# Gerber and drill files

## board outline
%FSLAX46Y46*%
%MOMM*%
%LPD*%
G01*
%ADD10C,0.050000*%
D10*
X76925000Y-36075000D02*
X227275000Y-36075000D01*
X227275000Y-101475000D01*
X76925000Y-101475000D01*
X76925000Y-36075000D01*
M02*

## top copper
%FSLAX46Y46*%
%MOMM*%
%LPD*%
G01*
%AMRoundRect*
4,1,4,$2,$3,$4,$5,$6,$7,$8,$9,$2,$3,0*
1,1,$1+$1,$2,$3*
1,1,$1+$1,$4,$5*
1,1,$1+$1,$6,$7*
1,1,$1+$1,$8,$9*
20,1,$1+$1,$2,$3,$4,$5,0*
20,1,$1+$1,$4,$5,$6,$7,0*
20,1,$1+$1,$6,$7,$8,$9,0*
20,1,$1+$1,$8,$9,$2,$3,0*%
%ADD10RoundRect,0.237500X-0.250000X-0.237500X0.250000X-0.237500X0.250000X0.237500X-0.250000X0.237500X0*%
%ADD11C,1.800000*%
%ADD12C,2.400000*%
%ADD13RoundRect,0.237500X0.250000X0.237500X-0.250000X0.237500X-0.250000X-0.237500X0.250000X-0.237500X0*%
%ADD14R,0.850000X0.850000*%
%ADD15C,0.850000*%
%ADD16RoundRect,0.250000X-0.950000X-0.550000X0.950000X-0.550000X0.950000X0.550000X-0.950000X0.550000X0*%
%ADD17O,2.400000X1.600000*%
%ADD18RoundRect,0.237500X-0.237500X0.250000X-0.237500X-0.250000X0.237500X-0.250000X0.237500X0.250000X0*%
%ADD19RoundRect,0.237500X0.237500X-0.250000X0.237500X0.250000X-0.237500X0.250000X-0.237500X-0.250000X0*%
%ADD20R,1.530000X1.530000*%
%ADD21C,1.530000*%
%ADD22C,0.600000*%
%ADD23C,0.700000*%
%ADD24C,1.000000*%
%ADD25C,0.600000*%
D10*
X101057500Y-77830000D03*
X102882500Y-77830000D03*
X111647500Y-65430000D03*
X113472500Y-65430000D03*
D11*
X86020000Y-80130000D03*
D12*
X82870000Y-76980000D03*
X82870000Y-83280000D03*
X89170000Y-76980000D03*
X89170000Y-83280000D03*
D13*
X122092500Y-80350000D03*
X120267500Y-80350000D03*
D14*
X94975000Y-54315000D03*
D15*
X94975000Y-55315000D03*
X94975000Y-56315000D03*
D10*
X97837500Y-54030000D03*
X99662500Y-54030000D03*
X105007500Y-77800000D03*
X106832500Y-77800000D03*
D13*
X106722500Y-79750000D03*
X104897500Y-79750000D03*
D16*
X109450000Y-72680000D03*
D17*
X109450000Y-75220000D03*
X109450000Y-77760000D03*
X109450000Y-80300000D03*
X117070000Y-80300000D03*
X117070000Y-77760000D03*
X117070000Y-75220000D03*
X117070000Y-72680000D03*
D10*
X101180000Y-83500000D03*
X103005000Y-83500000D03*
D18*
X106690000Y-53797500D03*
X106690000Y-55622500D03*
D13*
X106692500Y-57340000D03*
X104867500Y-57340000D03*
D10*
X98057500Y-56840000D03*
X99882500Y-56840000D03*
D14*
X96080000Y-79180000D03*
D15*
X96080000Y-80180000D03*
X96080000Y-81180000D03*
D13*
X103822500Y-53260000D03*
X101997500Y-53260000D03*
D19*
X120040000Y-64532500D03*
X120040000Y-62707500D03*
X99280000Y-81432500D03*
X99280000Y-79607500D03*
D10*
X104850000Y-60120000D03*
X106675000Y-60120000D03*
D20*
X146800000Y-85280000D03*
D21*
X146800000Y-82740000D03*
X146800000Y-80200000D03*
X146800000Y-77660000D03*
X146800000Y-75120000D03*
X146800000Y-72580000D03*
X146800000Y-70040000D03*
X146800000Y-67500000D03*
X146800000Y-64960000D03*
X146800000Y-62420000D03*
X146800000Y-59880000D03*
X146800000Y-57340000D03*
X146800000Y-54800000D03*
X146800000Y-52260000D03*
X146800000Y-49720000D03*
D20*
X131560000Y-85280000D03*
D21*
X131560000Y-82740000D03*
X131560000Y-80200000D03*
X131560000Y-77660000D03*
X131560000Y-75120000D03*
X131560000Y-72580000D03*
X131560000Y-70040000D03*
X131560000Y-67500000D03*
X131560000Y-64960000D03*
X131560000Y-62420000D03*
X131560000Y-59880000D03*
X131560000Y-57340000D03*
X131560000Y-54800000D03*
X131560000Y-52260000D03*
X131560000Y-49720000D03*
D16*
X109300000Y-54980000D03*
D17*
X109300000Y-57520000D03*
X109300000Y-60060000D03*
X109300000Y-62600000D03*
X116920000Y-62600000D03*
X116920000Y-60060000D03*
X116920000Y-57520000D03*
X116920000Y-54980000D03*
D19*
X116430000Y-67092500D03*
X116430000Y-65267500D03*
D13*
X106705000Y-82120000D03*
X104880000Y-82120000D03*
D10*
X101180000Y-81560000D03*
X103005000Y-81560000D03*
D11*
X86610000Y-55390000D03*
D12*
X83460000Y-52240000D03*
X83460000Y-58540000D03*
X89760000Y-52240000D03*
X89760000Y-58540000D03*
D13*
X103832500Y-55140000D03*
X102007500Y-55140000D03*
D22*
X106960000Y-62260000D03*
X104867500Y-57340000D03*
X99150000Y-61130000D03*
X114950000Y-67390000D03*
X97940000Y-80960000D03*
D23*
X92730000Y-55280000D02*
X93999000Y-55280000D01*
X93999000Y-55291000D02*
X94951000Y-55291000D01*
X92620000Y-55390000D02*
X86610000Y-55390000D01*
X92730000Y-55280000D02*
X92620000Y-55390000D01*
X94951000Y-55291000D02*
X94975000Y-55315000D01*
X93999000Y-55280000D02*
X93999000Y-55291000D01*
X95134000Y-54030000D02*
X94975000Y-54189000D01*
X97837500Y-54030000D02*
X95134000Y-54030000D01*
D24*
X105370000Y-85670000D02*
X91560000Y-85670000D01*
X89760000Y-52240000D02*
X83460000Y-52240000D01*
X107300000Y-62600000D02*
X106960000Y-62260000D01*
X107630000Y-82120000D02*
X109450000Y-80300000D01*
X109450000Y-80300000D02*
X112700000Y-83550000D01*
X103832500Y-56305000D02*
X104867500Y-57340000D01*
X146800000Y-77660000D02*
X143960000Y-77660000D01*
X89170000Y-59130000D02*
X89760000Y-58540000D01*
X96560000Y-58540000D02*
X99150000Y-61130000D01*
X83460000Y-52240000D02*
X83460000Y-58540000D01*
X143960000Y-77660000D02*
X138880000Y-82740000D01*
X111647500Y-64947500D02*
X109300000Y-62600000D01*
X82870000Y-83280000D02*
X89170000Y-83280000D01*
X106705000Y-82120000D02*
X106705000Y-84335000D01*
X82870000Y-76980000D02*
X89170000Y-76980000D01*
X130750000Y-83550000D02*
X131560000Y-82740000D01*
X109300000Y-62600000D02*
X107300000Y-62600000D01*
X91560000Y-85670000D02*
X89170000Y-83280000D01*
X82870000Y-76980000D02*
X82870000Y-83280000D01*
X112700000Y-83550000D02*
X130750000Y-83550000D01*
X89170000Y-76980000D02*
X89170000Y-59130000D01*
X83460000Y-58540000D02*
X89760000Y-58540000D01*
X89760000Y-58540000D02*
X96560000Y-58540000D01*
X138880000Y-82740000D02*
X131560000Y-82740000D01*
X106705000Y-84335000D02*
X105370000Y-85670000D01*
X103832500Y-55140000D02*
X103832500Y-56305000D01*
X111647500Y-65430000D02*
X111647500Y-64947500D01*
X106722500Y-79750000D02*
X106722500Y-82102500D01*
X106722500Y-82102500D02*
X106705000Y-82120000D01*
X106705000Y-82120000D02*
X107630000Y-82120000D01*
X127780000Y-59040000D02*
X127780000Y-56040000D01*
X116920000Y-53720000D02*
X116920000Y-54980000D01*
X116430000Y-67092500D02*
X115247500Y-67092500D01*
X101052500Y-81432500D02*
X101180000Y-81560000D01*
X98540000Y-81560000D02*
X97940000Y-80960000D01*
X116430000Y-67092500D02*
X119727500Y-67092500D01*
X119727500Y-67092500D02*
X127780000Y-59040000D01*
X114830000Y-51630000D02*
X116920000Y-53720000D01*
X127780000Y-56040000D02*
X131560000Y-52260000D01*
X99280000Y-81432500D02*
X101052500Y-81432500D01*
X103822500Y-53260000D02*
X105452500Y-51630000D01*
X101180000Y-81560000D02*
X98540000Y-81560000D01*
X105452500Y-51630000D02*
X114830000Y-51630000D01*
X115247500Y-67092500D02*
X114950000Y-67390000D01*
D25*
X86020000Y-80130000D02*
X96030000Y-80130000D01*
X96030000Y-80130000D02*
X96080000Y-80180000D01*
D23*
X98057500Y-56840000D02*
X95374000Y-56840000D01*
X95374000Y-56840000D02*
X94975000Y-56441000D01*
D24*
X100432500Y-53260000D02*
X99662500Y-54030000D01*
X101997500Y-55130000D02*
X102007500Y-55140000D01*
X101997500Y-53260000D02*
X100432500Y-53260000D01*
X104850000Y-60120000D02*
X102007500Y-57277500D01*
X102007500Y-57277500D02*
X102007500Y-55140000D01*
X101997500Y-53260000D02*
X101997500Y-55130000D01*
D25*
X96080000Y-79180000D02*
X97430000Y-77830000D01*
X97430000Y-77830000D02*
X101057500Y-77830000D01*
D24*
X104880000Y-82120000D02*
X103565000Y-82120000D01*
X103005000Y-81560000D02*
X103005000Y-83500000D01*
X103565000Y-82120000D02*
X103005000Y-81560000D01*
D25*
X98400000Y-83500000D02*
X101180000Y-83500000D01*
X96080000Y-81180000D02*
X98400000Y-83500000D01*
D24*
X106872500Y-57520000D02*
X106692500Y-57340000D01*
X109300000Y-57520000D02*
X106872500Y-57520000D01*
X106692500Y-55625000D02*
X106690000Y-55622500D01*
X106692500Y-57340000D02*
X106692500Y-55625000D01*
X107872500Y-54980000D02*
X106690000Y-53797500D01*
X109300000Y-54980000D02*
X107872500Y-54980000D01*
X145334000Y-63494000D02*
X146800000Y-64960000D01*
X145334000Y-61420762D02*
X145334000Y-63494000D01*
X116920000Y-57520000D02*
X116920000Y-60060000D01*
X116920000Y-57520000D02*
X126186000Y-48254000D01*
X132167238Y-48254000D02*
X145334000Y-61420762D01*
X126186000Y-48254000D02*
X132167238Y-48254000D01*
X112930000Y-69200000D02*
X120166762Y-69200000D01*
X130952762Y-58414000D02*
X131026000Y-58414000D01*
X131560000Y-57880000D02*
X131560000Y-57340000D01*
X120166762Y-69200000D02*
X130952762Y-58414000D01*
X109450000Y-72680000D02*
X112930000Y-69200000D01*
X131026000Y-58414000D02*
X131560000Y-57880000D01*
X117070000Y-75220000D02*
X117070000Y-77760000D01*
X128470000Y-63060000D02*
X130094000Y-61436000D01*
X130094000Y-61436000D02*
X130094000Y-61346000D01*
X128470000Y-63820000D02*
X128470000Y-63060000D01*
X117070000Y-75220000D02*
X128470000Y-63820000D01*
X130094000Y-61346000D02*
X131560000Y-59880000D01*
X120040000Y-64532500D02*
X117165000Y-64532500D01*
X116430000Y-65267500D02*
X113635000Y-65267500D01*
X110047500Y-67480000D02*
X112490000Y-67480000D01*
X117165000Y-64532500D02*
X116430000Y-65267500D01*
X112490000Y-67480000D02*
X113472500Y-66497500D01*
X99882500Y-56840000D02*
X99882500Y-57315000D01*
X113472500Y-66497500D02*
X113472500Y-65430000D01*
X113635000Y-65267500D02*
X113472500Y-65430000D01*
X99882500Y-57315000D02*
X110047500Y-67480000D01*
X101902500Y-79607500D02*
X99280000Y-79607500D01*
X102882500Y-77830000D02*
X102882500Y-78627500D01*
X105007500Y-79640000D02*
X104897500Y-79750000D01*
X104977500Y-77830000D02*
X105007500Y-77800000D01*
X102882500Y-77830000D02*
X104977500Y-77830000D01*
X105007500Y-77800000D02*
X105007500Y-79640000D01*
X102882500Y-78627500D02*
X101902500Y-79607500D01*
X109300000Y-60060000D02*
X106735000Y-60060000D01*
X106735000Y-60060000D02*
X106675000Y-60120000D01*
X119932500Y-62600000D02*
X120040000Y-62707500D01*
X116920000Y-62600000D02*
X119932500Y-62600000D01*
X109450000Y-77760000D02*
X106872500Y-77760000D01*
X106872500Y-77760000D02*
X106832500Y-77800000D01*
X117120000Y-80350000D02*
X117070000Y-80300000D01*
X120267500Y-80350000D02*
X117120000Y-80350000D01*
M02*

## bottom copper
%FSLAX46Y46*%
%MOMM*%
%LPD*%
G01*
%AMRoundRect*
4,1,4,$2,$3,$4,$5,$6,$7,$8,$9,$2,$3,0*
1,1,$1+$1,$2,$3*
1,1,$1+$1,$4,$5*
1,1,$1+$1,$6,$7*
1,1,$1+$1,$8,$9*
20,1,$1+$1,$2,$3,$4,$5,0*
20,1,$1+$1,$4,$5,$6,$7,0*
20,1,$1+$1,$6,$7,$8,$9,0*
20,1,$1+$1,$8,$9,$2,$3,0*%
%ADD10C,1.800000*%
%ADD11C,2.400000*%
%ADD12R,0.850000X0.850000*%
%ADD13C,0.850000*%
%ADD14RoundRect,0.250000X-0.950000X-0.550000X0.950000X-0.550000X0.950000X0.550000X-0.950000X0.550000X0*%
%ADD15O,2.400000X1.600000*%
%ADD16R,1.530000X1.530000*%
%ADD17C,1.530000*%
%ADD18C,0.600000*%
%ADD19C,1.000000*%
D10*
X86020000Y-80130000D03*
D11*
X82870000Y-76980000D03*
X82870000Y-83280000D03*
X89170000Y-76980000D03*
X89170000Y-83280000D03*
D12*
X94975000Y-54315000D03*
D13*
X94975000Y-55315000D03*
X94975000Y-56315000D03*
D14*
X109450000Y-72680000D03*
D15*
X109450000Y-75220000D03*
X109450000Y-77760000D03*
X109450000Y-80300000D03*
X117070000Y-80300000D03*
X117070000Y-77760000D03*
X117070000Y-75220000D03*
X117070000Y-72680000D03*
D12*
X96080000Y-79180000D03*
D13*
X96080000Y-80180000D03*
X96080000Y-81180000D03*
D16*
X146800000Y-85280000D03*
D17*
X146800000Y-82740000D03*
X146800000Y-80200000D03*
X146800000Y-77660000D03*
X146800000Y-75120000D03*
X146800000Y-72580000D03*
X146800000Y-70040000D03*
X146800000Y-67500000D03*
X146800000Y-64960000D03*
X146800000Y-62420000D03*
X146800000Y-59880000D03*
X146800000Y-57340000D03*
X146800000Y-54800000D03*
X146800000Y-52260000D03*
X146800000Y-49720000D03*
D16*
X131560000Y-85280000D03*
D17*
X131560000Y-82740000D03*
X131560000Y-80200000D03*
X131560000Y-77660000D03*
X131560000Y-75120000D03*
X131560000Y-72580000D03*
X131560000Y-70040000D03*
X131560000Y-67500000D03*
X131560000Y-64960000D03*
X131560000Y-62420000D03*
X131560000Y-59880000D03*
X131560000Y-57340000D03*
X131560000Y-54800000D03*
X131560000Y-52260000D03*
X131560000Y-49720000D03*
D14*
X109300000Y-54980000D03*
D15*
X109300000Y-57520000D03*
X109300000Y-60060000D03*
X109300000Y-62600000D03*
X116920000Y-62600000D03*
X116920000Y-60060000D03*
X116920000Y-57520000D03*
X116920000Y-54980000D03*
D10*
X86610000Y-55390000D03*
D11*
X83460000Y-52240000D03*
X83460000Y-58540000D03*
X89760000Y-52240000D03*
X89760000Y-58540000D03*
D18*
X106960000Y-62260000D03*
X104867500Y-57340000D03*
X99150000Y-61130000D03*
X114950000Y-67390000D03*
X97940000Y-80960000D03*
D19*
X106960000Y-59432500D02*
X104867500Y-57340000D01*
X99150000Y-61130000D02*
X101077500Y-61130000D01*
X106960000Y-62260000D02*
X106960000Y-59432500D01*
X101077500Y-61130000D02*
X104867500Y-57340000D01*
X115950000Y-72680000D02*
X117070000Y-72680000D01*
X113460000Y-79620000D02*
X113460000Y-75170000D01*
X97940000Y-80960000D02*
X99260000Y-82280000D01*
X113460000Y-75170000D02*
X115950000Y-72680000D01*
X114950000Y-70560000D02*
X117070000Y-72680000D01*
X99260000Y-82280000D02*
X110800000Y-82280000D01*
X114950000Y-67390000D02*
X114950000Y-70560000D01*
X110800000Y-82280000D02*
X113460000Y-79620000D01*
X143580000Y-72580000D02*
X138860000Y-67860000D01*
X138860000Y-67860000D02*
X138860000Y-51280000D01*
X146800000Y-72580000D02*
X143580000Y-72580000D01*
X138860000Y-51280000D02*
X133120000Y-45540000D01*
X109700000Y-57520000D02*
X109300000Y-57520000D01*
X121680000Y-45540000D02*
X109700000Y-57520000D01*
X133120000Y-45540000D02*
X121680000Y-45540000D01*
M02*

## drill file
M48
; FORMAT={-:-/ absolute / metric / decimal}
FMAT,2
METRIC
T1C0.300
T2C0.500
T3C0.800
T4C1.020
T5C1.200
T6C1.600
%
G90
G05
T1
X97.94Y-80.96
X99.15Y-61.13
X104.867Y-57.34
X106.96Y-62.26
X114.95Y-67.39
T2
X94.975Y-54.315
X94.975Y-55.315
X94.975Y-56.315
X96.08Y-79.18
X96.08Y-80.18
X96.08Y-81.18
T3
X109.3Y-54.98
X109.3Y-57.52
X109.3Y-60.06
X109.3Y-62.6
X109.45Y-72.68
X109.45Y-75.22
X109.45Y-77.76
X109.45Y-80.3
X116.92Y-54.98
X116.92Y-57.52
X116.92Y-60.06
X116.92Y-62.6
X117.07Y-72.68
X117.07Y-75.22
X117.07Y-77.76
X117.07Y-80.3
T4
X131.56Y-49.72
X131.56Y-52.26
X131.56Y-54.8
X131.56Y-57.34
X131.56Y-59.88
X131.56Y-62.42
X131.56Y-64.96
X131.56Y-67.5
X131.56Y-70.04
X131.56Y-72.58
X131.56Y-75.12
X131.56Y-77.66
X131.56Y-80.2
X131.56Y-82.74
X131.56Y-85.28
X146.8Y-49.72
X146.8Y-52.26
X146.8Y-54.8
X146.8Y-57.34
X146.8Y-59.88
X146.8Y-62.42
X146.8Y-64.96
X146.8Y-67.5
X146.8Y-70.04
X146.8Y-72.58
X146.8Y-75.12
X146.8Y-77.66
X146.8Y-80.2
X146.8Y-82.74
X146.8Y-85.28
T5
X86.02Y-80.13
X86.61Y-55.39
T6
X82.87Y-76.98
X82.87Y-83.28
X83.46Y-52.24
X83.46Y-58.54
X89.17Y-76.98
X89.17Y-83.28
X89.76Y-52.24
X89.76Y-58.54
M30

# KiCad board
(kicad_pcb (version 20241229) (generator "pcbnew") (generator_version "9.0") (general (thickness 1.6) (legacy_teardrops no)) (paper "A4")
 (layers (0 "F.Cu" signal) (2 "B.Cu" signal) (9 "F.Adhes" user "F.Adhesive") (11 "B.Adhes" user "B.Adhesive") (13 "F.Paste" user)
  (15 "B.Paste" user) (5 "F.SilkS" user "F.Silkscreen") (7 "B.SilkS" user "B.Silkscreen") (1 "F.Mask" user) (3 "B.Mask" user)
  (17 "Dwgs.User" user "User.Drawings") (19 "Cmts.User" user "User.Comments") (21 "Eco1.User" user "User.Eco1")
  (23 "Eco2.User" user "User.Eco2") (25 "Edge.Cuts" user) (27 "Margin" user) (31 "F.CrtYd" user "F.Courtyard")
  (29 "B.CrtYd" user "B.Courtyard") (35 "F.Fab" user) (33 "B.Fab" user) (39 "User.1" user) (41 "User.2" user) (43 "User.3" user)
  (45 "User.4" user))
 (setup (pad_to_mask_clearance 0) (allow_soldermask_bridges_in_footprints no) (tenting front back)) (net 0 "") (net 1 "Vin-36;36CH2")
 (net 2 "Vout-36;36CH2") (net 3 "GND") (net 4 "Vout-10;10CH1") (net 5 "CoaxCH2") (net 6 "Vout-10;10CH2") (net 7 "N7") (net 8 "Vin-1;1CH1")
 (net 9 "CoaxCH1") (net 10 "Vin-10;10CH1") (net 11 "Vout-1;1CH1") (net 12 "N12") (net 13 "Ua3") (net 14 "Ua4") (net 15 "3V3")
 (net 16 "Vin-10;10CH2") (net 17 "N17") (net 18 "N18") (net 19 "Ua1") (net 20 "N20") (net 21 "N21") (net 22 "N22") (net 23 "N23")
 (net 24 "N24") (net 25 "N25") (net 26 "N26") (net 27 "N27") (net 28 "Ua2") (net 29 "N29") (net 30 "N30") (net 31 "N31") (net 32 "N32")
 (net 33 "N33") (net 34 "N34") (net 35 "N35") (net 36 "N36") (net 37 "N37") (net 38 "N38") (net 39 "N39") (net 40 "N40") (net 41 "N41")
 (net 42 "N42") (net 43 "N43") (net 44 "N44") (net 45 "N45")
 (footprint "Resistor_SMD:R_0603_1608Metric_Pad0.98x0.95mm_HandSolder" (layer "F.Cu") (at 101.97 77.83)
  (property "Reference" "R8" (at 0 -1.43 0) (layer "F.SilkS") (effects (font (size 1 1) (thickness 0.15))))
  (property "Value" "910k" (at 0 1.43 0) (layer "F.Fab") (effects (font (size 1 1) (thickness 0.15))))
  (pad "1" smd roundrect (at -0.9125 0) (size 0.975 0.95) (layers "F.Cu" "F.Mask" "F.Paste") (roundrect_rratio 0.25) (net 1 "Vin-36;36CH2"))
  (pad "2" smd roundrect (at 0.9125 0) (size 0.975 0.95) (layers "F.Cu" "F.Mask" "F.Paste") (roundrect_rratio 0.25) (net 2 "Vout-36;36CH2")))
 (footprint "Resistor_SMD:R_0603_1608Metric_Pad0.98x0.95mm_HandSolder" (layer "F.Cu") (at 112.56 65.43)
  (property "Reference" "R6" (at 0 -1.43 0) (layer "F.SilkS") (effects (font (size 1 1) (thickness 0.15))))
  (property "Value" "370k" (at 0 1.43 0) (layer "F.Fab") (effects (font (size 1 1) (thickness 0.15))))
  (pad "1" smd roundrect (at -0.9125 0) (size 0.975 0.95) (layers "F.Cu" "F.Mask" "F.Paste") (roundrect_rratio 0.25) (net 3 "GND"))
  (pad "2" smd roundrect (at 0.9125 0) (size 0.975 0.95) (layers "F.Cu" "F.Mask" "F.Paste") (roundrect_rratio 0.25) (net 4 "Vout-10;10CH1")))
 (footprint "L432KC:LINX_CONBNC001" (layer "F.Cu") (at 86.02 80.13)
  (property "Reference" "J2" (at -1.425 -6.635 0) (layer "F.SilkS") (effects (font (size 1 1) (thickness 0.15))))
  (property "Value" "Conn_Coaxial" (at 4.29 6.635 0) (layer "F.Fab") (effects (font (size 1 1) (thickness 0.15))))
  (pad "1" thru_hole circle (at 0 0) (size 1.8 1.8) (drill 1.2) (layers "*.Cu" "*.Mask") (remove_unused_layers no) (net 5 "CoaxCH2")
   (solder_mask_margin 0.102))
  (pad "2" thru_hole circle (at -3.15 -3.15) (size 2.4 2.4) (drill 1.6) (layers "*.Cu" "*.Mask") (remove_unused_layers no) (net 3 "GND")
   (solder_mask_margin 0.102))
  (pad "2" thru_hole circle (at -3.15 3.15) (size 2.4 2.4) (drill 1.6) (layers "*.Cu" "*.Mask") (remove_unused_layers no) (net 3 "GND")
   (solder_mask_margin 0.102))
  (pad "2" thru_hole circle (at 3.15 -3.15) (size 2.4 2.4) (drill 1.6) (layers "*.Cu" "*.Mask") (remove_unused_layers no) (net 3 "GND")
   (solder_mask_margin 0.102))
  (pad "2" thru_hole circle (at 3.15 3.15) (size 2.4 2.4) (drill 1.6) (layers "*.Cu" "*.Mask") (remove_unused_layers no) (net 3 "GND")
   (solder_mask_margin 0.102)))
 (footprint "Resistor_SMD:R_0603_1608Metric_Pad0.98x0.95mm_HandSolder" (layer "F.Cu") (at 121.18 80.35 180)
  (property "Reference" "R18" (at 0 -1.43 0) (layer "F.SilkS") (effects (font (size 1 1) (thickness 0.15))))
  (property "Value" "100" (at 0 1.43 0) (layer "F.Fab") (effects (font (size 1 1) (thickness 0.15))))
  (pad "1" smd roundrect (at -0.9125 0 180) (size 0.975 0.95) (layers "F.Cu" "F.Mask" "F.Paste") (roundrect_rratio 0.25)
   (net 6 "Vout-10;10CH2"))
  (pad "2" smd roundrect (at 0.9125 0 180) (size 0.975 0.95) (layers "F.Cu" "F.Mask" "F.Paste") (roundrect_rratio 0.25) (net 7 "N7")))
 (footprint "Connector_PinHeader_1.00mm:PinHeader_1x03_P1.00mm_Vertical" (layer "F.Cu") (at 94.975 54.315)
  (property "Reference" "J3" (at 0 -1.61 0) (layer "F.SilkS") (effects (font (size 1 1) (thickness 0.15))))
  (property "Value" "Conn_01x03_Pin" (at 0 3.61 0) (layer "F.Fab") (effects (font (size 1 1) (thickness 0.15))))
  (pad "1" thru_hole rect (at 0 0) (size 0.85 0.85) (drill 0.5) (layers "*.Cu" "*.Mask") (remove_unused_layers no) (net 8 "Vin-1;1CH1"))
  (pad "2" thru_hole circle (at 0 1) (size 0.85 0.85) (drill 0.5) (layers "*.Cu" "*.Mask") (remove_unused_layers no) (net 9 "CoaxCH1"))
  (pad "3" thru_hole circle (at 0 2) (size 0.85 0.85) (drill 0.5) (layers "*.Cu" "*.Mask") (remove_unused_layers no) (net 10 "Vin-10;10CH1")))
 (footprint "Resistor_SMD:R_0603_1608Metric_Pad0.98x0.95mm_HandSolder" (layer "F.Cu") (at 98.75 54.03)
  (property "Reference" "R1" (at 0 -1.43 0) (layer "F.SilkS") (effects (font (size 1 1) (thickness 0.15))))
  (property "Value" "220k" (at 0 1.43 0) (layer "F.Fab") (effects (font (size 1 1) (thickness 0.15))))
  (pad "1" smd roundrect (at -0.9125 0) (size 0.975 0.95) (layers "F.Cu" "F.Mask" "F.Paste") (roundrect_rratio 0.25) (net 8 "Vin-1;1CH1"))
  (pad "2" smd roundrect (at 0.9125 0) (size 0.975 0.95) (layers "F.Cu" "F.Mask" "F.Paste") (roundrect_rratio 0.25) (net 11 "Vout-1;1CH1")))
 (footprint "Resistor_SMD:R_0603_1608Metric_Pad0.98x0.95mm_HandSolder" (layer "F.Cu") (at 105.92 77.8)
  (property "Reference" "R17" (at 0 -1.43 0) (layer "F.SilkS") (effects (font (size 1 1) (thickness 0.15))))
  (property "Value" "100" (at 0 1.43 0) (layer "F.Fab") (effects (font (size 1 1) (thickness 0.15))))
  (pad "1" smd roundrect (at -0.9125 0) (size 0.975 0.95) (layers "F.Cu" "F.Mask" "F.Paste") (roundrect_rratio 0.25) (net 2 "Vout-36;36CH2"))
  (pad "2" smd roundrect (at 0.9125 0) (size 0.975 0.95) (layers "F.Cu" "F.Mask" "F.Paste") (roundrect_rratio 0.25) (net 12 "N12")))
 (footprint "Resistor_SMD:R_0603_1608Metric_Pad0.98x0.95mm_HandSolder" (layer "F.Cu") (at 105.81 79.75 180)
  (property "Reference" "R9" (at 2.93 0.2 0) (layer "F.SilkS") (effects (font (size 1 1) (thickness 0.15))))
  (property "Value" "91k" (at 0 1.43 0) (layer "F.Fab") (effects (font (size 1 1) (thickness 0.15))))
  (pad "1" smd roundrect (at -0.9125 0 180) (size 0.975 0.95) (layers "F.Cu" "F.Mask" "F.Paste") (roundrect_rratio 0.25) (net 3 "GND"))
  (pad "2" smd roundrect (at 0.9125 0 180) (size 0.975 0.95) (layers "F.Cu" "F.Mask" "F.Paste") (roundrect_rratio 0.25)
   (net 2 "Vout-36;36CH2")))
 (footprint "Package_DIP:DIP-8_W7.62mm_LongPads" (layer "F.Cu") (at 109.45 72.68)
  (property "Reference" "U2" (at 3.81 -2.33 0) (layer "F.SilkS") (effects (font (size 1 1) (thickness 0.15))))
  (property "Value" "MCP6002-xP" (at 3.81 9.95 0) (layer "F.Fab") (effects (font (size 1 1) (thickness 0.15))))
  (pad "1" thru_hole roundrect (at 0 0) (size 2.4 1.6) (drill 0.8) (layers "*.Cu" "*.Mask") (remove_unused_layers no)
   (roundrect_rratio 0.15625) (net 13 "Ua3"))
  (pad "2" thru_hole oval (at 0 2.54) (size 2.4 1.6) (drill 0.8) (layers "*.Cu" "*.Mask") (remove_unused_layers no) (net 13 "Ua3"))
  (pad "3" thru_hole oval (at 0 5.08) (size 2.4 1.6) (drill 0.8) (layers "*.Cu" "*.Mask") (remove_unused_layers no) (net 12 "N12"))
  (pad "4" thru_hole oval (at 0 7.62) (size 2.4 1.6) (drill 0.8) (layers "*.Cu" "*.Mask") (remove_unused_layers no) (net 3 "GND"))
  (pad "5" thru_hole oval (at 7.62 7.62) (size 2.4 1.6) (drill 0.8) (layers "*.Cu" "*.Mask") (remove_unused_layers no) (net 7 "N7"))
  (pad "6" thru_hole oval (at 7.62 5.08) (size 2.4 1.6) (drill 0.8) (layers "*.Cu" "*.Mask") (remove_unused_layers no) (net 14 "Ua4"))
  (pad "7" thru_hole oval (at 7.62 2.54) (size 2.4 1.6) (drill 0.8) (layers "*.Cu" "*.Mask") (remove_unused_layers no) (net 14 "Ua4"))
  (pad "8" thru_hole oval (at 7.62 0) (size 2.4 1.6) (drill 0.8) (layers "*.Cu" "*.Mask") (remove_unused_layers no) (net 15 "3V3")))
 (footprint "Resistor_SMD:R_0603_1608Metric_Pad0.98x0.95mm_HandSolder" (layer "F.Cu") (at 102.0925 83.5)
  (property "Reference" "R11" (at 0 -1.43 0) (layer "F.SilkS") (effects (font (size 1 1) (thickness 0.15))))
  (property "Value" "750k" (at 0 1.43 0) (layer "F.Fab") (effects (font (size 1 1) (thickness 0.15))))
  (pad "1" smd roundrect (at -0.9125 0) (size 0.975 0.95) (layers "F.Cu" "F.Mask" "F.Paste") (roundrect_rratio 0.25) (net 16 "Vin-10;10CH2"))
  (pad "2" smd roundrect (at 0.9125 0) (size 0.975 0.95) (layers "F.Cu" "F.Mask" "F.Paste") (roundrect_rratio 0.25) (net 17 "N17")))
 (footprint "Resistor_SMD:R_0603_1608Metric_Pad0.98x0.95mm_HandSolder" (layer "F.Cu") (at 106.69 54.71 -90)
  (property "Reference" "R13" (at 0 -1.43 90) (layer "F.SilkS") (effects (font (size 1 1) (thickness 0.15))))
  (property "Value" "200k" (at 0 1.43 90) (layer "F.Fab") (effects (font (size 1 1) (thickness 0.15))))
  (pad "1" smd roundrect (at -0.9125 0 270) (size 0.975 0.95) (layers "F.Cu" "F.Mask" "F.Paste") (roundrect_rratio 0.25) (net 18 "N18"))
  (pad "2" smd roundrect (at 0.9125 0 270) (size 0.975 0.95) (layers "F.Cu" "F.Mask" "F.Paste") (roundrect_rratio 0.25) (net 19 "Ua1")))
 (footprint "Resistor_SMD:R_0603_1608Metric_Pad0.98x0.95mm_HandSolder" (layer "F.Cu") (at 105.78 57.34 180)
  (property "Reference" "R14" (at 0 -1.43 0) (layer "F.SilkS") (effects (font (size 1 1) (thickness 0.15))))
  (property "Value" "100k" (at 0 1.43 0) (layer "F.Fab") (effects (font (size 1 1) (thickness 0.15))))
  (pad "1" smd roundrect (at -0.9125 0 180) (size 0.975 0.95) (layers "F.Cu" "F.Mask" "F.Paste") (roundrect_rratio 0.25) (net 19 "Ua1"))
  (pad "2" smd roundrect (at 0.9125 0 180) (size 0.975 0.95) (layers "F.Cu" "F.Mask" "F.Paste") (roundrect_rratio 0.25) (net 3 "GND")))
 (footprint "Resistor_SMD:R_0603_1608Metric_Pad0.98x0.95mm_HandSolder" (layer "F.Cu") (at 98.97 56.84)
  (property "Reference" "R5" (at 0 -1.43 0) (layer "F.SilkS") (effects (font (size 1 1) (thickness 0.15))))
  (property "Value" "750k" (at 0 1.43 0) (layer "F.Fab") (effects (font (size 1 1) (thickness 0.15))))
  (pad "1" smd roundrect (at -0.9125 0) (size 0.975 0.95) (layers "F.Cu" "F.Mask" "F.Paste") (roundrect_rratio 0.25) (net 10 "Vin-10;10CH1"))
  (pad "2" smd roundrect (at 0.9125 0) (size 0.975 0.95) (layers "F.Cu" "F.Mask" "F.Paste") (roundrect_rratio 0.25) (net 4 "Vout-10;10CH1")))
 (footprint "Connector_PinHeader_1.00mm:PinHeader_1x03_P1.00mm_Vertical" (layer "F.Cu") (at 96.08 79.18)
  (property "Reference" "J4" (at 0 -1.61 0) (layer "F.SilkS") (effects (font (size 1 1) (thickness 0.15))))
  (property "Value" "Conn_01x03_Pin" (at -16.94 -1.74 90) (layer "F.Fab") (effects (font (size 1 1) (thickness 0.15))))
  (pad "1" thru_hole rect (at 0 0) (size 0.85 0.85) (drill 0.5) (layers "*.Cu" "*.Mask") (remove_unused_layers no) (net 1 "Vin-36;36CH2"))
  (pad "2" thru_hole circle (at 0 1) (size 0.85 0.85) (drill 0.5) (layers "*.Cu" "*.Mask") (remove_unused_layers no) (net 5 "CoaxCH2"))
  (pad "3" thru_hole circle (at 0 2) (size 0.85 0.85) (drill 0.5) (layers "*.Cu" "*.Mask") (remove_unused_layers no) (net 16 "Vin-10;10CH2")))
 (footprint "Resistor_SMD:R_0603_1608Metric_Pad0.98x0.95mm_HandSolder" (layer "F.Cu") (at 102.91 53.26 180)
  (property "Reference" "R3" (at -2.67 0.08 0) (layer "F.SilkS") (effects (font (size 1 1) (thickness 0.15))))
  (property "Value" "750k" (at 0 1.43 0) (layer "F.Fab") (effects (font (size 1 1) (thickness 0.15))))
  (pad "1" smd roundrect (at -0.9125 0 180) (size 0.975 0.95) (layers "F.Cu" "F.Mask" "F.Paste") (roundrect_rratio 0.25) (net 15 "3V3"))
  (pad "2" smd roundrect (at 0.9125 0 180) (size 0.975 0.95) (layers "F.Cu" "F.Mask" "F.Paste") (roundrect_rratio 0.25)
   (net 11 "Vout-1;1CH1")))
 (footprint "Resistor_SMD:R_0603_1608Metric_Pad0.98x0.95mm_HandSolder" (layer "F.Cu") (at 120.04 63.62 90)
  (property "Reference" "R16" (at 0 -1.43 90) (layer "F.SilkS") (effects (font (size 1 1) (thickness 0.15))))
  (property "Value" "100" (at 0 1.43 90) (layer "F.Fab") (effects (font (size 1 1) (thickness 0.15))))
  (pad "1" smd roundrect (at -0.9125 0 90) (size 0.975 0.95) (layers "F.Cu" "F.Mask" "F.Paste") (roundrect_rratio 0.25)
   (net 4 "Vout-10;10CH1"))
  (pad "2" smd roundrect (at 0.9125 0 90) (size 0.975 0.95) (layers "F.Cu" "F.Mask" "F.Paste") (roundrect_rratio 0.25) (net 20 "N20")))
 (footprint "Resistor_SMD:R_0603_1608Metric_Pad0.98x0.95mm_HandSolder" (layer "F.Cu") (at 99.28 80.52 90)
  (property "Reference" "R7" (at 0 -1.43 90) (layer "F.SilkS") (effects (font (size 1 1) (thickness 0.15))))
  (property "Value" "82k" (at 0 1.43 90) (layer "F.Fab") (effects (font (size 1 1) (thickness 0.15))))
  (pad "1" smd roundrect (at -0.9125 0 90) (size 0.975 0.95) (layers "F.Cu" "F.Mask" "F.Paste") (roundrect_rratio 0.25) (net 15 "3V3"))
  (pad "2" smd roundrect (at 0.9125 0 90) (size 0.975 0.95) (layers "F.Cu" "F.Mask" "F.Paste") (roundrect_rratio 0.25)
   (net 2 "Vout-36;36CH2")))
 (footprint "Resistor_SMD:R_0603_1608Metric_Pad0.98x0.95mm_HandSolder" (layer "F.Cu") (at 105.7625 60.12)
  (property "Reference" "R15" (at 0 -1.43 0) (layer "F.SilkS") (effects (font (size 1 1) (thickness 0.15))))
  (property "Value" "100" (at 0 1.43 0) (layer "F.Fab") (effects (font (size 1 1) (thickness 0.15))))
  (pad "1" smd roundrect (at -0.9125 0) (size 0.975 0.95) (layers "F.Cu" "F.Mask" "F.Paste") (roundrect_rratio 0.25) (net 11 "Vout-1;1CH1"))
  (pad "2" smd roundrect (at 0.9125 0) (size 0.975 0.95) (layers "F.Cu" "F.Mask" "F.Paste") (roundrect_rratio 0.25) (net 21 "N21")))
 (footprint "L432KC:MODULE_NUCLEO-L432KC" (layer "F.Cu") (at 139.18 69.065 180)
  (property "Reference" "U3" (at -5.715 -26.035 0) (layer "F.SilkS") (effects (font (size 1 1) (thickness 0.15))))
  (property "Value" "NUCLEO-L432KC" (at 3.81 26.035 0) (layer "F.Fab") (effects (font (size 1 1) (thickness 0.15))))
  (pad "CN3_1" thru_hole rect (at -7.62 -16.215 180) (size 1.53 1.53) (drill 1.02) (layers "*.Cu" "*.Mask") (remove_unused_layers no)
   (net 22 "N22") (solder_mask_margin 0.102))
  (pad "CN3_2" thru_hole circle (at -7.62 -13.675 180) (size 1.53 1.53) (drill 1.02) (layers "*.Cu" "*.Mask") (remove_unused_layers no)
   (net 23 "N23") (solder_mask_margin 0.102))
  (pad "CN3_3" thru_hole circle (at -7.62 -11.135 180) (size 1.53 1.53) (drill 1.02) (layers "*.Cu" "*.Mask") (remove_unused_layers no)
   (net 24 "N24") (solder_mask_margin 0.102))
  (pad "CN3_4" thru_hole circle (at -7.62 -8.595 180) (size 1.53 1.53) (drill 1.02) (layers "*.Cu" "*.Mask") (remove_unused_layers no)
   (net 3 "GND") (solder_mask_margin 0.102))
  (pad "CN3_5" thru_hole circle (at -7.62 -6.055 180) (size 1.53 1.53) (drill 1.02) (layers "*.Cu" "*.Mask") (remove_unused_layers no)
   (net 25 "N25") (solder_mask_margin 0.102))
  (pad "CN3_6" thru_hole circle (at -7.62 -3.515 180) (size 1.53 1.53) (drill 1.02) (layers "*.Cu" "*.Mask") (remove_unused_layers no)
   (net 19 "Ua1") (solder_mask_margin 0.102))
  (pad "CN3_7" thru_hole circle (at -7.62 -0.975 180) (size 1.53 1.53) (drill 1.02) (layers "*.Cu" "*.Mask") (remove_unused_layers no)
   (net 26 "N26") (solder_mask_margin 0.102))
  (pad "CN3_8" thru_hole circle (at -7.62 1.565 180) (size 1.53 1.53) (drill 1.02) (layers "*.Cu" "*.Mask") (remove_unused_layers no)
   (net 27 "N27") (solder_mask_margin 0.102))
  (pad "CN3_9" thru_hole circle (at -7.62 4.105 180) (size 1.53 1.53) (drill 1.02) (layers "*.Cu" "*.Mask") (remove_unused_layers no)
   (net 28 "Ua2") (solder_mask_margin 0.102))
  (pad "CN3_10" thru_hole circle (at -7.62 6.645 180) (size 1.53 1.53) (drill 1.02) (layers "*.Cu" "*.Mask") (remove_unused_layers no)
   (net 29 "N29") (solder_mask_margin 0.102))
  (pad "CN3_11" thru_hole circle (at -7.62 9.185 180) (size 1.53 1.53) (drill 1.02) (layers "*.Cu" "*.Mask") (remove_unused_layers no)
   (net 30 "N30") (solder_mask_margin 0.102))
  (pad "CN3_12" thru_hole circle (at -7.62 11.725 180) (size 1.53 1.53) (drill 1.02) (layers "*.Cu" "*.Mask") (remove_unused_layers no)
   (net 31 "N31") (solder_mask_margin 0.102))
  (pad "CN3_13" thru_hole circle (at -7.62 14.265 180) (size 1.53 1.53) (drill 1.02) (layers "*.Cu" "*.Mask") (remove_unused_layers no)
   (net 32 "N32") (solder_mask_margin 0.102))
  (pad "CN3_14" thru_hole circle (at -7.62 16.805 180) (size 1.53 1.53) (drill 1.02) (layers "*.Cu" "*.Mask") (remove_unused_layers no)
   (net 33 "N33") (solder_mask_margin 0.102))
  (pad "CN3_15" thru_hole circle (at -7.62 19.345 180) (size 1.53 1.53) (drill 1.02) (layers "*.Cu" "*.Mask") (remove_unused_layers no)
   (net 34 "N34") (solder_mask_margin 0.102))
  (pad "CN4_1" thru_hole rect (at 7.62 -16.215 180) (size 1.53 1.53) (drill 1.02) (layers "*.Cu" "*.Mask") (remove_unused_layers no)
   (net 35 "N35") (solder_mask_margin 0.102))
  (pad "CN4_2" thru_hole circle (at 7.62 -13.675 180) (size 1.53 1.53) (drill 1.02) (layers "*.Cu" "*.Mask") (remove_unused_layers no)
   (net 3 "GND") (solder_mask_margin 0.102))
  (pad "CN4_3" thru_hole circle (at 7.62 -11.135 180) (size 1.53 1.53) (drill 1.02) (layers "*.Cu" "*.Mask") (remove_unused_layers no)
   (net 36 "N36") (solder_mask_margin 0.102))
  (pad "CN4_4" thru_hole circle (at 7.62 -8.595 180) (size 1.53 1.53) (drill 1.02) (layers "*.Cu" "*.Mask") (remove_unused_layers no)
   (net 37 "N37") (solder_mask_margin 0.102))
  (pad "CN4_5" thru_hole circle (at 7.62 -6.055 180) (size 1.53 1.53) (drill 1.02) (layers "*.Cu" "*.Mask") (remove_unused_layers no)
   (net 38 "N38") (solder_mask_margin 0.102))
  (pad "CN4_6" thru_hole circle (at 7.62 -3.515 180) (size 1.53 1.53) (drill 1.02) (layers "*.Cu" "*.Mask") (remove_unused_layers no)
   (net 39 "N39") (solder_mask_margin 0.102))
  (pad "CN4_7" thru_hole circle (at 7.62 -0.975 180) (size 1.53 1.53) (drill 1.02) (layers "*.Cu" "*.Mask") (remove_unused_layers no)
   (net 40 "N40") (solder_mask_margin 0.102))
  (pad "CN4_8" thru_hole circle (at 7.62 1.565 180) (size 1.53 1.53) (drill 1.02) (layers "*.Cu" "*.Mask") (remove_unused_layers no)
   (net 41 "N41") (solder_mask_margin 0.102))
  (pad "CN4_9" thru_hole circle (at 7.62 4.105 180) (size 1.53 1.53) (drill 1.02) (layers "*.Cu" "*.Mask") (remove_unused_layers no)
   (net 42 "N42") (solder_mask_margin 0.102))
  (pad "CN4_10" thru_hole circle (at 7.62 6.645 180) (size 1.53 1.53) (drill 1.02) (layers "*.Cu" "*.Mask") (remove_unused_layers no)
   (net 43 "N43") (solder_mask_margin 0.102))
  (pad "CN4_11" thru_hole circle (at 7.62 9.185 180) (size 1.53 1.53) (drill 1.02) (layers "*.Cu" "*.Mask") (remove_unused_layers no)
   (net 14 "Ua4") (solder_mask_margin 0.102))
  (pad "CN4_12" thru_hole circle (at 7.62 11.725 180) (size 1.53 1.53) (drill 1.02) (layers "*.Cu" "*.Mask") (remove_unused_layers no)
   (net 13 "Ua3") (solder_mask_margin 0.102))
  (pad "CN4_13" thru_hole circle (at 7.62 14.265 180) (size 1.53 1.53) (drill 1.02) (layers "*.Cu" "*.Mask") (remove_unused_layers no)
   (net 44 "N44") (solder_mask_margin 0.102))
  (pad "CN4_14" thru_hole circle (at 7.62 16.805 180) (size 1.53 1.53) (drill 1.02) (layers "*.Cu" "*.Mask") (remove_unused_layers no)
   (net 15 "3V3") (solder_mask_margin 0.102))
  (pad "CN4_15" thru_hole circle (at 7.62 19.345 180) (size 1.53 1.53) (drill 1.02) (layers "*.Cu" "*.Mask") (remove_unused_layers no)
   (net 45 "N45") (solder_mask_margin 0.102)))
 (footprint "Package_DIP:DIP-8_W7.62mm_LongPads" (layer "F.Cu") (at 109.3 54.98)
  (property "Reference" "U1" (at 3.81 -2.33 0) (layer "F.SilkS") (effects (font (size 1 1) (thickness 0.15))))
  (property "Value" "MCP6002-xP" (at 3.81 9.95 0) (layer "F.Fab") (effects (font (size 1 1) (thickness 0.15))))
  (pad "1" thru_hole roundrect (at 0 0) (size 2.4 1.6) (drill 0.8) (layers "*.Cu" "*.Mask") (remove_unused_layers no)
   (roundrect_rratio 0.15625) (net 18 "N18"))
  (pad "2" thru_hole oval (at 0 2.54) (size 2.4 1.6) (drill 0.8) (layers "*.Cu" "*.Mask") (remove_unused_layers no) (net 19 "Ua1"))
  (pad "3" thru_hole oval (at 0 5.08) (size 2.4 1.6) (drill 0.8) (layers "*.Cu" "*.Mask") (remove_unused_layers no) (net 21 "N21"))
  (pad "4" thru_hole oval (at 0 7.62) (size 2.4 1.6) (drill 0.8) (layers "*.Cu" "*.Mask") (remove_unused_layers no) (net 3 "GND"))
  (pad "5" thru_hole oval (at 7.62 7.62) (size 2.4 1.6) (drill 0.8) (layers "*.Cu" "*.Mask") (remove_unused_layers no) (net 20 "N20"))
  (pad "6" thru_hole oval (at 7.62 5.08) (size 2.4 1.6) (drill 0.8) (layers "*.Cu" "*.Mask") (remove_unused_layers no) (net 28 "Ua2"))
  (pad "7" thru_hole oval (at 7.62 2.54) (size 2.4 1.6) (drill 0.8) (layers "*.Cu" "*.Mask") (remove_unused_layers no) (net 28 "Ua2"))
  (pad "8" thru_hole oval (at 7.62 0) (size 2.4 1.6) (drill 0.8) (layers "*.Cu" "*.Mask") (remove_unused_layers no) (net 15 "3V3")))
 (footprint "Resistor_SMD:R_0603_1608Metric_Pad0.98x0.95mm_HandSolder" (layer "F.Cu") (at 116.43 66.18 90)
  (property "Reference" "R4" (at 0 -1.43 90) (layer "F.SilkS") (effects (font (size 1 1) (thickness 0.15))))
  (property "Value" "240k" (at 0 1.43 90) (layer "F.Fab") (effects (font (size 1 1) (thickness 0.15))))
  (pad "1" smd roundrect (at -0.9125 0 90) (size 0.975 0.95) (layers "F.Cu" "F.Mask" "F.Paste") (roundrect_rratio 0.25) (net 15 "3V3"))
  (pad "2" smd roundrect (at 0.9125 0 90) (size 0.975 0.95) (layers "F.Cu" "F.Mask" "F.Paste") (roundrect_rratio 0.25)
   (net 4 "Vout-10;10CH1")))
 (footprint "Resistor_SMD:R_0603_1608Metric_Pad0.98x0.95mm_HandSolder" (layer "F.Cu") (at 105.7925 82.12 180)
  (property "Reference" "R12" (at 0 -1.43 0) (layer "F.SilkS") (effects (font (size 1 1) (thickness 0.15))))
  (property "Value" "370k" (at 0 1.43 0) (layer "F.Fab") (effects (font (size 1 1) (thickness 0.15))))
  (pad "1" smd roundrect (at -0.9125 0 180) (size 0.975 0.95) (layers "F.Cu" "F.Mask" "F.Paste") (roundrect_rratio 0.25) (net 3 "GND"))
  (pad "2" smd roundrect (at 0.9125 0 180) (size 0.975 0.95) (layers "F.Cu" "F.Mask" "F.Paste") (roundrect_rratio 0.25) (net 17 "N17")))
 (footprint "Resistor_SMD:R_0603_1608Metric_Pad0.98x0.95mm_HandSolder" (layer "F.Cu") (at 102.0925 81.56)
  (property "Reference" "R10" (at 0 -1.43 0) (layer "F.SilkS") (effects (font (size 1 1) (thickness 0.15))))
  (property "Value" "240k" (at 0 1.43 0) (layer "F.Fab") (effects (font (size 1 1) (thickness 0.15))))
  (pad "1" smd roundrect (at -0.9125 0) (size 0.975 0.95) (layers "F.Cu" "F.Mask" "F.Paste") (roundrect_rratio 0.25) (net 15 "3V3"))
  (pad "2" smd roundrect (at 0.9125 0) (size 0.975 0.95) (layers "F.Cu" "F.Mask" "F.Paste") (roundrect_rratio 0.25) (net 17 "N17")))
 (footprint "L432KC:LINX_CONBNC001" (layer "F.Cu") (at 86.61 55.39)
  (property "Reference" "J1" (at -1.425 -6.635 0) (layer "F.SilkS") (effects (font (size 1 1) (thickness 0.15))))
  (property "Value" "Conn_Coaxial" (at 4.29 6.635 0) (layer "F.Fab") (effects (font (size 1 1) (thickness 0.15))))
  (pad "1" thru_hole circle (at 0 0) (size 1.8 1.8) (drill 1.2) (layers "*.Cu" "*.Mask") (remove_unused_layers no) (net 9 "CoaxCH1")
   (solder_mask_margin 0.102))
  (pad "2" thru_hole circle (at -3.15 -3.15) (size 2.4 2.4) (drill 1.6) (layers "*.Cu" "*.Mask") (remove_unused_layers no) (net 3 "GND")
   (solder_mask_margin 0.102))
  (pad "2" thru_hole circle (at -3.15 3.15) (size 2.4 2.4) (drill 1.6) (layers "*.Cu" "*.Mask") (remove_unused_layers no) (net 3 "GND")
   (solder_mask_margin 0.102))
  (pad "2" thru_hole circle (at 3.15 -3.15) (size 2.4 2.4) (drill 1.6) (layers "*.Cu" "*.Mask") (remove_unused_layers no) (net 3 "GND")
   (solder_mask_margin 0.102))
  (pad "2" thru_hole circle (at 3.15 3.15) (size 2.4 2.4) (drill 1.6) (layers "*.Cu" "*.Mask") (remove_unused_layers no) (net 3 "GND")
   (solder_mask_margin 0.102)))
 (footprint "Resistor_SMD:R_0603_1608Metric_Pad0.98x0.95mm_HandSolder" (layer "F.Cu") (at 102.92 55.14 180)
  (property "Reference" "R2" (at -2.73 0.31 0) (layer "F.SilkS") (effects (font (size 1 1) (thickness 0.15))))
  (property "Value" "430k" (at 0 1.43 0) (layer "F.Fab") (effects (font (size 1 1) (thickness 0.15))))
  (pad "1" smd roundrect (at -0.9125 0 180) (size 0.975 0.95) (layers "F.Cu" "F.Mask" "F.Paste") (roundrect_rratio 0.25) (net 3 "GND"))
  (pad "2" smd roundrect (at 0.9125 0 180) (size 0.975 0.95) (layers "F.Cu" "F.Mask" "F.Paste") (roundrect_rratio 0.25)
   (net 11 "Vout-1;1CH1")))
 (gr_rect (start 76.925 36.075) (end 227.275 101.475) (stroke (width 0.05) (type default)) (fill no) (layer "Edge.Cuts"))
 (segment (start 92.73 55.28) (end 93.999 55.28) (width 0.7) (layer "F.Cu") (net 9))
 (segment (start 93.999 55.291) (end 94.951 55.291) (width 0.7) (layer "F.Cu") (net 9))
 (segment (start 92.62 55.39) (end 86.61 55.39) (width 0.7) (layer "F.Cu") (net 9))
 (segment (start 92.73 55.28) (end 92.62 55.39) (width 0.7) (layer "F.Cu") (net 9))
 (segment (start 94.951 55.291) (end 94.975 55.315) (width 0.7) (layer "F.Cu") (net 9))
 (segment (start 93.999 55.28) (end 93.999 55.291) (width 0.7) (layer "F.Cu") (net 9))
 (segment (start 95.134 54.03) (end 94.975 54.189) (width 0.7) (layer "F.Cu") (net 8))
 (segment (start 97.8375 54.03) (end 95.134 54.03) (width 0.7) (layer "F.Cu") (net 8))
 (segment (start 105.37 85.67) (end 91.56 85.67) (width 1) (layer "F.Cu") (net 3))
 (segment (start 89.76 52.24) (end 83.46 52.24) (width 1) (layer "F.Cu") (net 3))
 (segment (start 107.3 62.6) (end 106.96 62.26) (width 1) (layer "F.Cu") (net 3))
 (segment (start 107.63 82.12) (end 109.45 80.3) (width 1) (layer "F.Cu") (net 3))
 (segment (start 109.45 80.3) (end 112.7 83.55) (width 1) (layer "F.Cu") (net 3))
 (segment (start 103.8325 56.305) (end 104.8675 57.34) (width 1) (layer "F.Cu") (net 3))
 (segment (start 146.8 77.66) (end 143.96 77.66) (width 1) (layer "F.Cu") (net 3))
 (segment (start 89.17 59.13) (end 89.76 58.54) (width 1) (layer "F.Cu") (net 3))
 (segment (start 96.56 58.54) (end 99.15 61.13) (width 1) (layer "F.Cu") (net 3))
 (segment (start 83.46 52.24) (end 83.46 58.54) (width 1) (layer "F.Cu") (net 3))
 (segment (start 143.96 77.66) (end 138.88 82.74) (width 1) (layer "F.Cu") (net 3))
 (segment (start 111.6475 64.9475) (end 109.3 62.6) (width 1) (layer "F.Cu") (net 3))
 (segment (start 82.87 83.28) (end 89.17 83.28) (width 1) (layer "F.Cu") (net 3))
 (segment (start 106.705 82.12) (end 106.705 84.335) (width 1) (layer "F.Cu") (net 3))
 (segment (start 82.87 76.98) (end 89.17 76.98) (width 1) (layer "F.Cu") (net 3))
 (segment (start 130.75 83.55) (end 131.56 82.74) (width 1) (layer "F.Cu") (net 3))
 (segment (start 109.3 62.6) (end 107.3 62.6) (width 1) (layer "F.Cu") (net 3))
 (segment (start 91.56 85.67) (end 89.17 83.28) (width 1) (layer "F.Cu") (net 3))
 (segment (start 82.87 76.98) (end 82.87 83.28) (width 1) (layer "F.Cu") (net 3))
 (segment (start 112.7 83.55) (end 130.75 83.55) (width 1) (layer "F.Cu") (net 3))
 (segment (start 89.17 76.98) (end 89.17 59.13) (width 1) (layer "F.Cu") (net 3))
 (segment (start 83.46 58.54) (end 89.76 58.54) (width 1) (layer "F.Cu") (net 3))
 (segment (start 89.76 58.54) (end 96.56 58.54) (width 1) (layer "F.Cu") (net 3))
 (segment (start 138.88 82.74) (end 131.56 82.74) (width 1) (layer "F.Cu") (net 3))
 (segment (start 106.705 84.335) (end 105.37 85.67) (width 1) (layer "F.Cu") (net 3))
 (segment (start 103.8325 55.14) (end 103.8325 56.305) (width 1) (layer "F.Cu") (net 3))
 (segment (start 111.6475 65.43) (end 111.6475 64.9475) (width 1) (layer "F.Cu") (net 3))
 (segment (start 106.7225 79.75) (end 106.7225 82.1025) (width 1) (layer "F.Cu") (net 3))
 (segment (start 106.7225 82.1025) (end 106.705 82.12) (width 1) (layer "F.Cu") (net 3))
 (segment (start 106.705 82.12) (end 107.63 82.12) (width 1) (layer "F.Cu") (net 3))
 (via (at 106.96 62.26) (size 0.6) (drill 0.3) (layers "F.Cu" "B.Cu") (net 3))
 (via (at 104.8675 57.34) (size 0.6) (drill 0.3) (layers "F.Cu" "B.Cu") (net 3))
 (via (at 99.15 61.13) (size 0.6) (drill 0.3) (layers "F.Cu" "B.Cu") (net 3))
 (segment (start 106.96 59.4325) (end 104.8675 57.34) (width 1) (layer "B.Cu") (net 3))
 (segment (start 99.15 61.13) (end 101.0775 61.13) (width 1) (layer "B.Cu") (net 3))
 (segment (start 106.96 62.26) (end 106.96 59.4325) (width 1) (layer "B.Cu") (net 3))
 (segment (start 101.0775 61.13) (end 104.8675 57.34) (width 1) (layer "B.Cu") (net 3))
 (segment (start 127.78 59.04) (end 127.78 56.04) (width 1) (layer "F.Cu") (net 15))
 (segment (start 116.92 53.72) (end 116.92 54.98) (width 1) (layer "F.Cu") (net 15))
 (segment (start 116.43 67.0925) (end 115.2475 67.0925) (width 1) (layer "F.Cu") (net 15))
 (segment (start 101.0525 81.4325) (end 101.18 81.56) (width 1) (layer "F.Cu") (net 15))
 (segment (start 98.54 81.56) (end 97.94 80.96) (width 1) (layer "F.Cu") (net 15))
 (segment (start 116.43 67.0925) (end 119.7275 67.0925) (width 1) (layer "F.Cu") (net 15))
 (segment (start 119.7275 67.0925) (end 127.78 59.04) (width 1) (layer "F.Cu") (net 15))
 (segment (start 114.83 51.63) (end 116.92 53.72) (width 1) (layer "F.Cu") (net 15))
 (segment (start 127.78 56.04) (end 131.56 52.26) (width 1) (layer "F.Cu") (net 15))
 (segment (start 99.28 81.4325) (end 101.0525 81.4325) (width 1) (layer "F.Cu") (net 15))
 (segment (start 103.8225 53.26) (end 105.4525 51.63) (width 1) (layer "F.Cu") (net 15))
 (segment (start 101.18 81.56) (end 98.54 81.56) (width 1) (layer "F.Cu") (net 15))
 (segment (start 105.4525 51.63) (end 114.83 51.63) (width 1) (layer "F.Cu") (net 15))
 (segment (start 115.2475 67.0925) (end 114.95 67.39) (width 1) (layer "F.Cu") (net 15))
 (via (at 114.95 67.39) (size 0.6) (drill 0.3) (layers "F.Cu" "B.Cu") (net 15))
 (via (at 97.94 80.96) (size 0.6) (drill 0.3) (layers "F.Cu" "B.Cu") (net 15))
 (segment (start 115.95 72.68) (end 117.07 72.68) (width 1) (layer "B.Cu") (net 15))
 (segment (start 113.46 79.62) (end 113.46 75.17) (width 1) (layer "B.Cu") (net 15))
 (segment (start 97.94 80.96) (end 99.26 82.28) (width 1) (layer "B.Cu") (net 15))
 (segment (start 113.46 75.17) (end 115.95 72.68) (width 1) (layer "B.Cu") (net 15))
 (segment (start 114.95 70.56) (end 117.07 72.68) (width 1) (layer "B.Cu") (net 15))
 (segment (start 99.26 82.28) (end 110.8 82.28) (width 1) (layer "B.Cu") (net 15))
 (segment (start 114.95 67.39) (end 114.95 70.56) (width 1) (layer "B.Cu") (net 15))
 (segment (start 110.8 82.28) (end 113.46 79.62) (width 1) (layer "B.Cu") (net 15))
 (segment (start 86.02 80.13) (end 96.03 80.13) (width 0.6) (layer "F.Cu") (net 5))
 (segment (start 96.03 80.13) (end 96.08 80.18) (width 0.6) (layer "F.Cu") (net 5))
 (segment (start 98.0575 56.84) (end 95.374 56.84) (width 0.7) (layer "F.Cu") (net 10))
 (segment (start 95.374 56.84) (end 94.975 56.441) (width 0.7) (layer "F.Cu") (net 10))
 (segment (start 100.4325 53.26) (end 99.6625 54.03) (width 1) (layer "F.Cu") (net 11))
 (segment (start 101.9975 55.13) (end 102.0075 55.14) (width 1) (layer "F.Cu") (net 11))
 (segment (start 101.9975 53.26) (end 100.4325 53.26) (width 1) (layer "F.Cu") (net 11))
 (segment (start 104.85 60.12) (end 102.0075 57.2775) (width 1) (layer "F.Cu") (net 11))
 (segment (start 102.0075 57.2775) (end 102.0075 55.14) (width 1) (layer "F.Cu") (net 11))
 (segment (start 101.9975 53.26) (end 101.9975 55.13) (width 1) (layer "F.Cu") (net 11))
 (segment (start 96.08 79.18) (end 97.43 77.83) (width 0.6) (layer "F.Cu") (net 1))
 (segment (start 97.43 77.83) (end 101.0575 77.83) (width 0.6) (layer "F.Cu") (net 1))
 (segment (start 104.88 82.12) (end 103.565 82.12) (width 1) (layer "F.Cu") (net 17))
 (segment (start 103.005 81.56) (end 103.005 83.5) (width 1) (layer "F.Cu") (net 17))
 (segment (start 103.565 82.12) (end 103.005 81.56) (width 1) (layer "F.Cu") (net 17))
 (segment (start 98.4 83.5) (end 101.18 83.5) (width 0.6) (layer "F.Cu") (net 16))
 (segment (start 96.08 81.18) (end 98.4 83.5) (width 0.6) (layer "F.Cu") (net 16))
 (segment (start 106.8725 57.52) (end 106.6925 57.34) (width 1) (layer "F.Cu") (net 19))
 (segment (start 109.3 57.52) (end 106.8725 57.52) (width 1) (layer "F.Cu") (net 19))
 (segment (start 106.6925 55.625) (end 106.69 55.6225) (width 1) (layer "F.Cu") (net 19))
 (segment (start 106.6925 57.34) (end 106.6925 55.625) (width 1) (layer "F.Cu") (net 19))
 (segment (start 143.58 72.58) (end 138.86 67.86) (width 1) (layer "B.Cu") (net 19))
 (segment (start 138.86 67.86) (end 138.86 51.28) (width 1) (layer "B.Cu") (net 19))
 (segment (start 146.8 72.58) (end 143.58 72.58) (width 1) (layer "B.Cu") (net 19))
 (segment (start 138.86 51.28) (end 133.12 45.54) (width 1) (layer "B.Cu") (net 19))
 (segment (start 109.7 57.52) (end 109.3 57.52) (width 1) (layer "B.Cu") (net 19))
 (segment (start 121.68 45.54) (end 109.7 57.52) (width 1) (layer "B.Cu") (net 19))
 (segment (start 133.12 45.54) (end 121.68 45.54) (width 1) (layer "B.Cu") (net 19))
 (segment (start 107.8725 54.98) (end 106.69 53.7975) (width 1) (layer "F.Cu") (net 18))
 (segment (start 109.3 54.98) (end 107.8725 54.98) (width 1) (layer "F.Cu") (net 18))
 (segment (start 145.334 63.494) (end 146.8 64.96) (width 1) (layer "F.Cu") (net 28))
 (segment (start 145.334 61.420762) (end 145.334 63.494) (width 1) (layer "F.Cu") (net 28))
 (segment (start 116.92 57.52) (end 116.92 60.06) (width 1) (layer "F.Cu") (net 28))
 (segment (start 116.92 57.52) (end 126.186 48.254) (width 1) (layer "F.Cu") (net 28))
 (segment (start 132.167238 48.254) (end 145.334 61.420762) (width 1) (layer "F.Cu") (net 28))
 (segment (start 126.186 48.254) (end 132.167238 48.254) (width 1) (layer "F.Cu") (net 28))
 (segment (start 112.93 69.2) (end 120.166762 69.2) (width 1) (layer "F.Cu") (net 13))
 (segment (start 130.952762 58.414) (end 131.026 58.414) (width 1) (layer "F.Cu") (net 13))
 (segment (start 131.56 57.88) (end 131.56 57.34) (width 1) (layer "F.Cu") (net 13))
 (segment (start 120.166762 69.2) (end 130.952762 58.414) (width 1) (layer "F.Cu") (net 13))
 (segment (start 109.45 72.68) (end 112.93 69.2) (width 1) (layer "F.Cu") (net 13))
 (segment (start 131.026 58.414) (end 131.56 57.88) (width 1) (layer "F.Cu") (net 13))
 (segment (start 117.07 75.22) (end 117.07 77.76) (width 1) (layer "F.Cu") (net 14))
 (segment (start 128.47 63.06) (end 130.094 61.436) (width 1) (layer "F.Cu") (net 14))
 (segment (start 130.094 61.436) (end 130.094 61.346) (width 1) (layer "F.Cu") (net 14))
 (segment (start 128.47 63.82) (end 128.47 63.06) (width 1) (layer "F.Cu") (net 14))
 (segment (start 117.07 75.22) (end 128.47 63.82) (width 1) (layer "F.Cu") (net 14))
 (segment (start 130.094 61.346) (end 131.56 59.88) (width 1) (layer "F.Cu") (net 14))
 (segment (start 120.04 64.5325) (end 117.165 64.5325) (width 1) (layer "F.Cu") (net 4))
 (segment (start 116.43 65.2675) (end 113.635 65.2675) (width 1) (layer "F.Cu") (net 4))
 (segment (start 110.0475 67.48) (end 112.49 67.48) (width 1) (layer "F.Cu") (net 4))
 (segment (start 117.165 64.5325) (end 116.43 65.2675) (width 1) (layer "F.Cu") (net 4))
 (segment (start 112.49 67.48) (end 113.4725 66.4975) (width 1) (layer "F.Cu") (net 4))
 (segment (start 99.8825 56.84) (end 99.8825 57.315) (width 1) (layer "F.Cu") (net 4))
 (segment (start 113.4725 66.4975) (end 113.4725 65.43) (width 1) (layer "F.Cu") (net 4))
 (segment (start 113.635 65.2675) (end 113.4725 65.43) (width 1) (layer "F.Cu") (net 4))
 (segment (start 99.8825 57.315) (end 110.0475 67.48) (width 1) (layer "F.Cu") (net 4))
 (segment (start 101.9025 79.6075) (end 99.28 79.6075) (width 1) (layer "F.Cu") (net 2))
 (segment (start 102.8825 77.83) (end 102.8825 78.6275) (width 1) (layer "F.Cu") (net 2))
 (segment (start 105.0075 79.64) (end 104.8975 79.75) (width 1) (layer "F.Cu") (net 2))
 (segment (start 104.9775 77.83) (end 105.0075 77.8) (width 1) (layer "F.Cu") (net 2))
 (segment (start 102.8825 77.83) (end 104.9775 77.83) (width 1) (layer "F.Cu") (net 2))
 (segment (start 105.0075 77.8) (end 105.0075 79.64) (width 1) (layer "F.Cu") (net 2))
 (segment (start 102.8825 78.6275) (end 101.9025 79.6075) (width 1) (layer "F.Cu") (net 2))
 (segment (start 109.3 60.06) (end 106.735 60.06) (width 1) (layer "F.Cu") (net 21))
 (segment (start 106.735 60.06) (end 106.675 60.12) (width 1) (layer "F.Cu") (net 21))
 (segment (start 119.9325 62.6) (end 120.04 62.7075) (width 1) (layer "F.Cu") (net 20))
 (segment (start 116.92 62.6) (end 119.9325 62.6) (width 1) (layer "F.Cu") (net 20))
 (segment (start 109.45 77.76) (end 106.8725 77.76) (width 1) (layer "F.Cu") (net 12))
 (segment (start 106.8725 77.76) (end 106.8325 77.8) (width 1) (layer "F.Cu") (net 12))
 (segment (start 117.12 80.35) (end 117.07 80.3) (width 1) (layer "F.Cu") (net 7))
 (segment (start 120.2675 80.35) (end 117.12 80.35) (width 1) (layer "F.Cu") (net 7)))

